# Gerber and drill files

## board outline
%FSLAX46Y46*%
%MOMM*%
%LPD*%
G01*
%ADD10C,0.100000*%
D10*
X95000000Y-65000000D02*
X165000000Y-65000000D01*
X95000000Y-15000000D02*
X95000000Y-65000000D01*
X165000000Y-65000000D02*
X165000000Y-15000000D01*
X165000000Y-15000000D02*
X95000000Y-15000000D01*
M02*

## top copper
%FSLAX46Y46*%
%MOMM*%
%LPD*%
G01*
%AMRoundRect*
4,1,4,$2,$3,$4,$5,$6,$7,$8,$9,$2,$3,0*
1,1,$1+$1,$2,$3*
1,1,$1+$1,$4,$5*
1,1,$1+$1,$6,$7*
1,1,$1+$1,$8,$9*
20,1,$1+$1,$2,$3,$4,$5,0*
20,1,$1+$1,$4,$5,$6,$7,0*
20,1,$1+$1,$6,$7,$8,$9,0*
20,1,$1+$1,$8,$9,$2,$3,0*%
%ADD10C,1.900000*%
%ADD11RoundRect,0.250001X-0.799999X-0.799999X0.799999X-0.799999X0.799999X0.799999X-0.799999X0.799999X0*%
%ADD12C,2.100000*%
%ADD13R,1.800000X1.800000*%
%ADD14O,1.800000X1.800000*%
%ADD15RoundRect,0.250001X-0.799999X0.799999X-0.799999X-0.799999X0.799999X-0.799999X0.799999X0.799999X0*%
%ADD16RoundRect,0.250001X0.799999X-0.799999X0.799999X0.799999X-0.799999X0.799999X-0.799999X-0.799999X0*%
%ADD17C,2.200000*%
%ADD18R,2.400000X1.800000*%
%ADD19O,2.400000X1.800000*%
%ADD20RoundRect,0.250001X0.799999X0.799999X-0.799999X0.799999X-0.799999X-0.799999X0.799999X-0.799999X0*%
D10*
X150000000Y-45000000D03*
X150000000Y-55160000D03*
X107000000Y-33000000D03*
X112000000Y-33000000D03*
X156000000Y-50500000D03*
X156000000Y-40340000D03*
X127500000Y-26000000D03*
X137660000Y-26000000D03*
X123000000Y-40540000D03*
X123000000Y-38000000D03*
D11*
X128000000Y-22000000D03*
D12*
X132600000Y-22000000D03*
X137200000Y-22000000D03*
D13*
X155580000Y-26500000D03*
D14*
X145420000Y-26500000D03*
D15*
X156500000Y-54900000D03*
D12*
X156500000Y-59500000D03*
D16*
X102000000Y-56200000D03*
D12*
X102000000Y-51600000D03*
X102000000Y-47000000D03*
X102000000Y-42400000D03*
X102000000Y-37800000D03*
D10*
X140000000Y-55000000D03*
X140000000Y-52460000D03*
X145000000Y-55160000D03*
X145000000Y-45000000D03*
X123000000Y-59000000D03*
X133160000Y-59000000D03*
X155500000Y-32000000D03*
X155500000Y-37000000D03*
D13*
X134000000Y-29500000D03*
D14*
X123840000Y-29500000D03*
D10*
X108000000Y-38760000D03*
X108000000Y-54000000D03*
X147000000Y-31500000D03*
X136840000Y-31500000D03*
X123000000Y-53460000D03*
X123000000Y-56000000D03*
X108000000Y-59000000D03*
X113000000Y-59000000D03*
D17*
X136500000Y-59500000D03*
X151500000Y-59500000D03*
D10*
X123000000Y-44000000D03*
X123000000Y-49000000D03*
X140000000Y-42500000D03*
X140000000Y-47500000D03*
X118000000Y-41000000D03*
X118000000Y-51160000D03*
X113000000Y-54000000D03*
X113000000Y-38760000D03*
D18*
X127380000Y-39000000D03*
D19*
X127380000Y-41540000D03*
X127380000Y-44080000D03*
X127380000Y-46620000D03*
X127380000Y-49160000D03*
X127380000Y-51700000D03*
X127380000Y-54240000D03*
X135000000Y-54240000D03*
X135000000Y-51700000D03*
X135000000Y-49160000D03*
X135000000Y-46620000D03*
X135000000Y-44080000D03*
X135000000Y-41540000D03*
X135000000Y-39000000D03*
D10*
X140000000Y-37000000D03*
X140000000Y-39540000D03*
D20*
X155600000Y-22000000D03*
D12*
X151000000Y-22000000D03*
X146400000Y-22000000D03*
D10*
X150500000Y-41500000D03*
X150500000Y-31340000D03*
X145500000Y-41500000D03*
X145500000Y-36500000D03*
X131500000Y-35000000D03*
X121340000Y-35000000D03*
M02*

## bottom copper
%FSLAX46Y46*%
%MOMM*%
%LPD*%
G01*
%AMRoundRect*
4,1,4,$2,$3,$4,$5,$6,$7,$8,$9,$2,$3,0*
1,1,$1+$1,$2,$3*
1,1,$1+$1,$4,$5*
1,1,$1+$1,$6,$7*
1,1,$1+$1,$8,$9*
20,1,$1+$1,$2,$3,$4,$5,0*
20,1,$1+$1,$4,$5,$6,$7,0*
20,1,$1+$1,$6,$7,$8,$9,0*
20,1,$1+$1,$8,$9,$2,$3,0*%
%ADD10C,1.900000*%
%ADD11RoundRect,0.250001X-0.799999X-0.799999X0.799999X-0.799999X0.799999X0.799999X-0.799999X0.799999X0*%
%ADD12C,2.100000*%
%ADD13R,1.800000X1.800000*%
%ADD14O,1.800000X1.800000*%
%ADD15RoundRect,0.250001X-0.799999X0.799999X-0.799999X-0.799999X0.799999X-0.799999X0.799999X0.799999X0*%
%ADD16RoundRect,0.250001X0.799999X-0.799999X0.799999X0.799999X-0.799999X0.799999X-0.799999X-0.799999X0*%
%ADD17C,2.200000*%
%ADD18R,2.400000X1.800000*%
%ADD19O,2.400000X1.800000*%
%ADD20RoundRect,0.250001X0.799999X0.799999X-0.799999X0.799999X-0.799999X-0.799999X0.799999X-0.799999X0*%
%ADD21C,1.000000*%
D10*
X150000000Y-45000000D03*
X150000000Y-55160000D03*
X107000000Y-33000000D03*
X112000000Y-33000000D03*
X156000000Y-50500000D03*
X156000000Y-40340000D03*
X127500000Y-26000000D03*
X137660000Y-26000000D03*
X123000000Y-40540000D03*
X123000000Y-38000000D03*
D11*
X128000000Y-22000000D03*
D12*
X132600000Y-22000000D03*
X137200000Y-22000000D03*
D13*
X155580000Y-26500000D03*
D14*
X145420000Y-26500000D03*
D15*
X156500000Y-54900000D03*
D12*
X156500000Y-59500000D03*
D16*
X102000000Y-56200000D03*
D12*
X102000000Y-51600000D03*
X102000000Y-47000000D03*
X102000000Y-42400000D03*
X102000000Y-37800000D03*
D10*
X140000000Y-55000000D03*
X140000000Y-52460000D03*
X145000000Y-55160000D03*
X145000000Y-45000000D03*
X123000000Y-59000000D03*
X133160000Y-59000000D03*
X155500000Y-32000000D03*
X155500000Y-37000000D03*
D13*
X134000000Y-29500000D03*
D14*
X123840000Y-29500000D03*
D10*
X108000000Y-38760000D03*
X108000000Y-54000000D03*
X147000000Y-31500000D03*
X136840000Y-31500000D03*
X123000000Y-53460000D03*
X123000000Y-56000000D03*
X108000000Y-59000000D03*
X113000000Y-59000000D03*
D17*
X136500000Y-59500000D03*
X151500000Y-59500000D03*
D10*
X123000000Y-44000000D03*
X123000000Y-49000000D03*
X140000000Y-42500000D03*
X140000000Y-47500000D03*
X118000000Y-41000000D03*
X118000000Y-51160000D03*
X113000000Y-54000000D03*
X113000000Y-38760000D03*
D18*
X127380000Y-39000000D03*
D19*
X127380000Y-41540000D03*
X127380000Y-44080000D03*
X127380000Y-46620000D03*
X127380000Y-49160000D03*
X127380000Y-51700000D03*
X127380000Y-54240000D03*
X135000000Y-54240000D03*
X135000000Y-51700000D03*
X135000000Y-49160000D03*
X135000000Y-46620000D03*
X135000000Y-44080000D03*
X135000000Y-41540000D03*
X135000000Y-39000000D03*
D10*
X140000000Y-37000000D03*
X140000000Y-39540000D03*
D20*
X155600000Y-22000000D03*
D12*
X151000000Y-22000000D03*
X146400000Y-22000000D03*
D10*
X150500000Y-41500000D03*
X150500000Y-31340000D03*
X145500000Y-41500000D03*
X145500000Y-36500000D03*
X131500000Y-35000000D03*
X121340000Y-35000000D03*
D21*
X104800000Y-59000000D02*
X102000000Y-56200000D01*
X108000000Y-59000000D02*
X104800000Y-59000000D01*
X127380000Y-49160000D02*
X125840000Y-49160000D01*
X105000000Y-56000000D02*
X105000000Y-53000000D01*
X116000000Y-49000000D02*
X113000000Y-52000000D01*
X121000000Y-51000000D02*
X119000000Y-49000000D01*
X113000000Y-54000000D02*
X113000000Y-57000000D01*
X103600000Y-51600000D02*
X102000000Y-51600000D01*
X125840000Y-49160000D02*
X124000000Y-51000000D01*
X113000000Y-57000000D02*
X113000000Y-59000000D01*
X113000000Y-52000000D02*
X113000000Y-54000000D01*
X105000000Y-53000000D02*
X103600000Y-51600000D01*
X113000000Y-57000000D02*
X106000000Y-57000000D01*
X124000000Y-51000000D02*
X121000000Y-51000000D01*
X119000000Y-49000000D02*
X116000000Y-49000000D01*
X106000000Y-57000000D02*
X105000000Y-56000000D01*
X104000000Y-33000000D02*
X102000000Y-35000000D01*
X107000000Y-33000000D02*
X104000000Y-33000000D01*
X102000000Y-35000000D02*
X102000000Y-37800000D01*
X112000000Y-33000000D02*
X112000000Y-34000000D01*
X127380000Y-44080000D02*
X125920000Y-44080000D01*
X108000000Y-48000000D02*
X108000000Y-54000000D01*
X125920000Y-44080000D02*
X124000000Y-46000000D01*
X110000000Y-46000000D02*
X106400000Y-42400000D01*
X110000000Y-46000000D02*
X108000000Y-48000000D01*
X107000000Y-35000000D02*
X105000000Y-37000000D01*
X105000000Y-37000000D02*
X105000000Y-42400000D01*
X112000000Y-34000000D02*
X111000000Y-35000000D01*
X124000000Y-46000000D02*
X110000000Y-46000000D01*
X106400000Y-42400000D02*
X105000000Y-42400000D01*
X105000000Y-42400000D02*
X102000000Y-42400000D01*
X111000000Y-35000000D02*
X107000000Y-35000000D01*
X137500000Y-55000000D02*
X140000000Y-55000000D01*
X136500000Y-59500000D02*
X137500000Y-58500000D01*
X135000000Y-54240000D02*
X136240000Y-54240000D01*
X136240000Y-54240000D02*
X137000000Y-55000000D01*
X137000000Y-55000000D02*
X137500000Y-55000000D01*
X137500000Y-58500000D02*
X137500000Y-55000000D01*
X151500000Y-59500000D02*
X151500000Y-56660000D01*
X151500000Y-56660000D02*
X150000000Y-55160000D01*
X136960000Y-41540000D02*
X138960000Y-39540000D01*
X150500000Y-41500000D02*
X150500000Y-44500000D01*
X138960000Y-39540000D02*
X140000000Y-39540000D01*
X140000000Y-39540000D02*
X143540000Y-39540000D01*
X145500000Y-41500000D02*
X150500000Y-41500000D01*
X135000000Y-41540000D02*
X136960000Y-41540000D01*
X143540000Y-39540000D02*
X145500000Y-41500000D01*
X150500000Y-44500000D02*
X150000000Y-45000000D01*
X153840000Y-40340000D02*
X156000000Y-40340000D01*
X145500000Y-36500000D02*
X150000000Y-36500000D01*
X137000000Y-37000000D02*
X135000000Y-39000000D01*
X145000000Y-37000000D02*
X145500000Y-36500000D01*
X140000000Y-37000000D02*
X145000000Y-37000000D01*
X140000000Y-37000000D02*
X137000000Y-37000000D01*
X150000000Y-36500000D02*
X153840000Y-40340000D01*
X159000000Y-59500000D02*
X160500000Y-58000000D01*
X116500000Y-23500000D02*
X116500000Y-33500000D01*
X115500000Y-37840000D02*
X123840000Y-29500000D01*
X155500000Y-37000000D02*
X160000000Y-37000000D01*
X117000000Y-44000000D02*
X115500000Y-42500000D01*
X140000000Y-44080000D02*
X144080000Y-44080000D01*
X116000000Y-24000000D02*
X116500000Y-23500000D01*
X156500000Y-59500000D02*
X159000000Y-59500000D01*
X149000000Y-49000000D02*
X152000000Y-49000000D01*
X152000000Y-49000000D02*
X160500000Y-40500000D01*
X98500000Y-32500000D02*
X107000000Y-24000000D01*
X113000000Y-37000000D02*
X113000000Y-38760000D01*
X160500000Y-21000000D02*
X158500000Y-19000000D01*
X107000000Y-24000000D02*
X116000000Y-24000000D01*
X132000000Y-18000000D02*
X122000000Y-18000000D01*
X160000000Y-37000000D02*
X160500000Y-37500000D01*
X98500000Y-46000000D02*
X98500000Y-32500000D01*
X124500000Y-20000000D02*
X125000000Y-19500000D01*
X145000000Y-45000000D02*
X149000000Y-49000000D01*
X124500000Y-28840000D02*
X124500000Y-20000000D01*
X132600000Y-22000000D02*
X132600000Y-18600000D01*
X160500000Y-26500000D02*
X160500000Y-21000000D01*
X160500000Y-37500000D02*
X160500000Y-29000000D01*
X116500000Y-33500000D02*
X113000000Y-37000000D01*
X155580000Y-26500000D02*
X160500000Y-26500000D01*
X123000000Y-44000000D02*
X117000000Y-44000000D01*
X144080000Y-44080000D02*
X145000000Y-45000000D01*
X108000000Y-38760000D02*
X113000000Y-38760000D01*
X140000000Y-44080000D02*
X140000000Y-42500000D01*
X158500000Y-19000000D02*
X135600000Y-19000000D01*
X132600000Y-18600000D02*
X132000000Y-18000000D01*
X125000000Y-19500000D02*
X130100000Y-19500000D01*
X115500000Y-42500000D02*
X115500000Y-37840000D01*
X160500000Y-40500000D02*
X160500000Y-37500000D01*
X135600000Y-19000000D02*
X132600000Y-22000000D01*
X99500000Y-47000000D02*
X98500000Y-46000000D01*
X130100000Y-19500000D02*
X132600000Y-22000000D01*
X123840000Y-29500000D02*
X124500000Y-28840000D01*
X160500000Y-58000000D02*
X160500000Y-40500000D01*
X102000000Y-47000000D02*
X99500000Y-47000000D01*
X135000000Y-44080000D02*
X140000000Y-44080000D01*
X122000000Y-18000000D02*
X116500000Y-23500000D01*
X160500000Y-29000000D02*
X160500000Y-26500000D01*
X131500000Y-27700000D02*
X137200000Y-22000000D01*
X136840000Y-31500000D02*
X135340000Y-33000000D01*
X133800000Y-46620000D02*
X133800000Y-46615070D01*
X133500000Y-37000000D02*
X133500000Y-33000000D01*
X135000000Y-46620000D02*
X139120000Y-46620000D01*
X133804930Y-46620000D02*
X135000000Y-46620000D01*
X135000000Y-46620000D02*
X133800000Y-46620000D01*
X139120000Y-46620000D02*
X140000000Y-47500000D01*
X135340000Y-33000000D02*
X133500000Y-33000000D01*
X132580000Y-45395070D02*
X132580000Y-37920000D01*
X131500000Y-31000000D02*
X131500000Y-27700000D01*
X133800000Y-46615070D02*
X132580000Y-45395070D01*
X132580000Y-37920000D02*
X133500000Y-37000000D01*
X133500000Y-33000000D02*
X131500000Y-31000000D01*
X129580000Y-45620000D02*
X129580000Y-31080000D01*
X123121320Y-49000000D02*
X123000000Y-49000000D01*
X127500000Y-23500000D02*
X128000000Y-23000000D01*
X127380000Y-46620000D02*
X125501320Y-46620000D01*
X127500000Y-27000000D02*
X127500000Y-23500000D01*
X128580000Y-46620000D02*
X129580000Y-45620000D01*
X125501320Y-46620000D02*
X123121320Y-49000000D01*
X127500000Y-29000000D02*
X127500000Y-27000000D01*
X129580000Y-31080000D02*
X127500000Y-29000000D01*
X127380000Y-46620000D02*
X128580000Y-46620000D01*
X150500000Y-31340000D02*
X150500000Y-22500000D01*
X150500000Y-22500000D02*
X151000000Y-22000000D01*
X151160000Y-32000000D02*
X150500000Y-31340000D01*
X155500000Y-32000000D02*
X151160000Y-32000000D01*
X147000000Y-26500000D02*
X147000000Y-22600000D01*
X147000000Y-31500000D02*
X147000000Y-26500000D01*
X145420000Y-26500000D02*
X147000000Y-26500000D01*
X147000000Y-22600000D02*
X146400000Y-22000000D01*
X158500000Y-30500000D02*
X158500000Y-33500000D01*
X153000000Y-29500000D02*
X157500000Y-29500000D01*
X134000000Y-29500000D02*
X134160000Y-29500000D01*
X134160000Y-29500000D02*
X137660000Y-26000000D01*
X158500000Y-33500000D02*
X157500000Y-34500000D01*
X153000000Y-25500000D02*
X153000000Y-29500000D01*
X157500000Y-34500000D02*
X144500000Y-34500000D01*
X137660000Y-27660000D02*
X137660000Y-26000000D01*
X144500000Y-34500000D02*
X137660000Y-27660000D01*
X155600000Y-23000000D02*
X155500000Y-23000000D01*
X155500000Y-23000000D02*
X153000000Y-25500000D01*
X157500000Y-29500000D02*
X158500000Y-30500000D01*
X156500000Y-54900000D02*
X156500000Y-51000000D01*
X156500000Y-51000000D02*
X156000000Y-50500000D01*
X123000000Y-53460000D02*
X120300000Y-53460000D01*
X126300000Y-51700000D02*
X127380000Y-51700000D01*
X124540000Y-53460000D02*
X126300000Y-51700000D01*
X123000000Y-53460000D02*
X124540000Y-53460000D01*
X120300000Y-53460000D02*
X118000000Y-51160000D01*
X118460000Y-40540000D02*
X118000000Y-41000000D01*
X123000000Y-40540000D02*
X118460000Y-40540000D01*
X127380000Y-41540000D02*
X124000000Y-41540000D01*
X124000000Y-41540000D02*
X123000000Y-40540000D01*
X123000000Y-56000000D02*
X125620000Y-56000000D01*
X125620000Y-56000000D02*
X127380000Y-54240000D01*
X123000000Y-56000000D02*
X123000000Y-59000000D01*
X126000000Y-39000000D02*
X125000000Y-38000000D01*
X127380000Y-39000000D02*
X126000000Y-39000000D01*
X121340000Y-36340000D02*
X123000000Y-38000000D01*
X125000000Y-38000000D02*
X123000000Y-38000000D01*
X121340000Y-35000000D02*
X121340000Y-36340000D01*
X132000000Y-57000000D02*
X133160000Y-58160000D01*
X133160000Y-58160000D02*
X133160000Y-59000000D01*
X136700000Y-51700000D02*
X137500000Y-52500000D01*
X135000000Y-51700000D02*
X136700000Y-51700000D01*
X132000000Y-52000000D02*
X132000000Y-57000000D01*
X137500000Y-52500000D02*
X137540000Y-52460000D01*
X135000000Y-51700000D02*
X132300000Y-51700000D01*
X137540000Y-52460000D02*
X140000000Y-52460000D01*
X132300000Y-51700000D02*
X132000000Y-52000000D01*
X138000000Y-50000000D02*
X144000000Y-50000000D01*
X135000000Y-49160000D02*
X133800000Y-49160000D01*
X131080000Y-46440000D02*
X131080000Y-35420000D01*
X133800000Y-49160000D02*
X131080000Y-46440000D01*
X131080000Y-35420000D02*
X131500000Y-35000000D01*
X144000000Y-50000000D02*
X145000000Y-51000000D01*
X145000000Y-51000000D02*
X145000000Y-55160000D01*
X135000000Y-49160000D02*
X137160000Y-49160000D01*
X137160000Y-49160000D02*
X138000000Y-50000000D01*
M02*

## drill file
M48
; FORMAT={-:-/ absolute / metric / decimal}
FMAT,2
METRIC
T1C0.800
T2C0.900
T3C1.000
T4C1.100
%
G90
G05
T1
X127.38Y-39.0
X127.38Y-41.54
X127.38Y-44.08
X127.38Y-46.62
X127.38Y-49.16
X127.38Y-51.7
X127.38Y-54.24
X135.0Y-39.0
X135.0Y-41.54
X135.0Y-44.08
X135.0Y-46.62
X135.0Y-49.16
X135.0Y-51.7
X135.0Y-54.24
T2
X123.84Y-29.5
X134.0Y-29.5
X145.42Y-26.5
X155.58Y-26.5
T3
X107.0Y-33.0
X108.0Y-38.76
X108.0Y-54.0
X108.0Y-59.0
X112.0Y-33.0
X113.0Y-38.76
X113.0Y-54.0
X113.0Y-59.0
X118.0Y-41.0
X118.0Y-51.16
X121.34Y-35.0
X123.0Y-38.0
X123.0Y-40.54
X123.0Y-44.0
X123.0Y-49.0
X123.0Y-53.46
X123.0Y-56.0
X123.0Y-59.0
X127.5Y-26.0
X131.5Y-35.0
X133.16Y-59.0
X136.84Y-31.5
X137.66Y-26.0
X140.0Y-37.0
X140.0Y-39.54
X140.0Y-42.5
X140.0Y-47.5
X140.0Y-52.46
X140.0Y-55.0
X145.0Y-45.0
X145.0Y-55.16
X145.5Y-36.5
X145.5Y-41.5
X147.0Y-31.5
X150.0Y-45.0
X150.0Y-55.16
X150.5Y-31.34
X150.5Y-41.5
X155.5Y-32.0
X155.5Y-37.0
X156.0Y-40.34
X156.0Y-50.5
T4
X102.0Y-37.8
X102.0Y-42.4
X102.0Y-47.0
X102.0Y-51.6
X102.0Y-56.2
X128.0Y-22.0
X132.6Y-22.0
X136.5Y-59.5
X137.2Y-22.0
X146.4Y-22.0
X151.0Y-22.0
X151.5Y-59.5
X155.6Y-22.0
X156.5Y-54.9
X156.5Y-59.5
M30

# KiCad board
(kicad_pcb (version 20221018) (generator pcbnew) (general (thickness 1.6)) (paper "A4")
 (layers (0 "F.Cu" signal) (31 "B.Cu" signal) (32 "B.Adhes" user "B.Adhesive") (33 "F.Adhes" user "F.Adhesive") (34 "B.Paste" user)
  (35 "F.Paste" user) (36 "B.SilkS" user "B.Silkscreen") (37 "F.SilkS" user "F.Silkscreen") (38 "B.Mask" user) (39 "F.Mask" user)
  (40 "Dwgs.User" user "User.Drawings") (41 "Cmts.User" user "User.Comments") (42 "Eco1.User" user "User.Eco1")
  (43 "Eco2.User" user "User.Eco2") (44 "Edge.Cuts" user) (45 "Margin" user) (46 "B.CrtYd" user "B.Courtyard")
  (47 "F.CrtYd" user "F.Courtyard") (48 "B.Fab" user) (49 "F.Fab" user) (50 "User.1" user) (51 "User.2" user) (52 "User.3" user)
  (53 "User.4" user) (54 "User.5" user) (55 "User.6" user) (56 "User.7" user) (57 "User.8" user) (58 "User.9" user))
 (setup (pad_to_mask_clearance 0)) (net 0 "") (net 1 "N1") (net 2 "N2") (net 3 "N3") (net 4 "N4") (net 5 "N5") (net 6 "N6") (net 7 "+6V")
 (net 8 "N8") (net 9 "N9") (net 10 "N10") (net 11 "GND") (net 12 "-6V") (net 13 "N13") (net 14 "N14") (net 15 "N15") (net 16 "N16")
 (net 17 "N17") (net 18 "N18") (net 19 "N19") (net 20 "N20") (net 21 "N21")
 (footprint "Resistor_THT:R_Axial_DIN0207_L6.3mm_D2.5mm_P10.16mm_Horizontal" (layer "F.Cu") (at 150 45 -90)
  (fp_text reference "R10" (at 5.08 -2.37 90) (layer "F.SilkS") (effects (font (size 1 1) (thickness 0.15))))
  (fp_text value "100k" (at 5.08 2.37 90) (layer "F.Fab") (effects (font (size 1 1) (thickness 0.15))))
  (pad "1" thru_hole circle (at 0 0 270) (size 1.9 1.9) (drill 1) (layers "*.Cu" "*.Mask") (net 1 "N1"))
  (pad "2" thru_hole circle (at 10.16 0 270) (size 1.9 1.9) (drill 1) (layers "*.Cu" "*.Mask") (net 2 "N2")))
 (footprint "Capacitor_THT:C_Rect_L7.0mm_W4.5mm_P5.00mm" (layer "F.Cu") (at 107 33)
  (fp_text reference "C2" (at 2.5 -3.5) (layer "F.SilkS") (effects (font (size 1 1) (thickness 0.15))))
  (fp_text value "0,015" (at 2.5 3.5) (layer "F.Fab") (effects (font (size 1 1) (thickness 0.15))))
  (pad "1" thru_hole circle (at 0 0) (size 1.9 1.9) (drill 1) (layers "*.Cu" "*.Mask") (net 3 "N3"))
  (pad "2" thru_hole circle (at 5 0) (size 1.9 1.9) (drill 1) (layers "*.Cu" "*.Mask") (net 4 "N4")))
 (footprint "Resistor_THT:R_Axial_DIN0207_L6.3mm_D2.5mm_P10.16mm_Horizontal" (layer "F.Cu") (at 156 50.5 90)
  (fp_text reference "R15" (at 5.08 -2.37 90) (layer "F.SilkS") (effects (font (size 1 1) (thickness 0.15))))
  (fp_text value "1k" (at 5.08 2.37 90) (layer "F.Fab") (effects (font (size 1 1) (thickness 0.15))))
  (pad "1" thru_hole circle (at 0 0 90) (size 1.9 1.9) (drill 1) (layers "*.Cu" "*.Mask") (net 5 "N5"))
  (pad "2" thru_hole circle (at 10.16 0 90) (size 1.9 1.9) (drill 1) (layers "*.Cu" "*.Mask") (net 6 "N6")))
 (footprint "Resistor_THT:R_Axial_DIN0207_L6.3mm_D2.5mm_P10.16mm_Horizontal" (layer "F.Cu") (at 127.5 26)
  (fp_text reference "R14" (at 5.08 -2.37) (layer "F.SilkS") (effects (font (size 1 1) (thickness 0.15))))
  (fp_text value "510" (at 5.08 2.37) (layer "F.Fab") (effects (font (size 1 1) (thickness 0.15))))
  (pad "1" thru_hole circle (at 0 0) (size 1.9 1.9) (drill 1) (layers "*.Cu" "*.Mask") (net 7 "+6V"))
  (pad "2" thru_hole circle (at 10.16 0) (size 1.9 1.9) (drill 1) (layers "*.Cu" "*.Mask") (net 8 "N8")))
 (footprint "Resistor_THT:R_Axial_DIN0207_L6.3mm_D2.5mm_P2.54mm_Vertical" (layer "F.Cu") (at 123 40.54 90)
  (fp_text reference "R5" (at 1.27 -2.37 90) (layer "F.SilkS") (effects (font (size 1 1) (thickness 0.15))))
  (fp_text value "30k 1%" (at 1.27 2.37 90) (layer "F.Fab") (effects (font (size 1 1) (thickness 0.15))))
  (pad "1" thru_hole circle (at 0 0 90) (size 1.9 1.9) (drill 1) (layers "*.Cu" "*.Mask") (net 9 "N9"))
  (pad "2" thru_hole circle (at 2.54 0 90) (size 1.9 1.9) (drill 1) (layers "*.Cu" "*.Mask") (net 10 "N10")))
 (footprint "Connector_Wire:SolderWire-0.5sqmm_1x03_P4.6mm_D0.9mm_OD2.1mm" (layer "F.Cu") (at 128 22)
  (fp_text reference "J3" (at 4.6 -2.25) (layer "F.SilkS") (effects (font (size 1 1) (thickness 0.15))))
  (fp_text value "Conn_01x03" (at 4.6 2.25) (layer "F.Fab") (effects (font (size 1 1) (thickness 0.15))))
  (pad "1" thru_hole roundrect (at 0 0) (size 2.1 2.1) (drill 1.1) (layers "*.Cu" "*.Mask") (roundrect_rratio 0.119048) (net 7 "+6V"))
  (pad "2" thru_hole circle (at 4.6 0) (size 2.1 2.1) (drill 1.1) (layers "*.Cu" "*.Mask") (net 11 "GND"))
  (pad "3" thru_hole circle (at 9.2 0) (size 2.1 2.1) (drill 1.1) (layers "*.Cu" "*.Mask") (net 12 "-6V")))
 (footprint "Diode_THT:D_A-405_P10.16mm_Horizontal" (layer "F.Cu") (at 155.58 26.5 180)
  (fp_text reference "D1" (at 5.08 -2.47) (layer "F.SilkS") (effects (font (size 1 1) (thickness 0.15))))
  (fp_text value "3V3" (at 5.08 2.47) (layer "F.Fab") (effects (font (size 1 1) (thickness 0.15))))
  (pad "1" thru_hole rect (at 0 0 180) (size 1.8 1.8) (drill 0.9) (layers "*.Cu" "*.Mask") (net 11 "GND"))
  (pad "2" thru_hole oval (at 10.16 0 180) (size 1.8 1.8) (drill 0.9) (layers "*.Cu" "*.Mask") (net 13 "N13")))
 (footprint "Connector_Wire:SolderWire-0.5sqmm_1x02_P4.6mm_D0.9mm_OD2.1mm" (layer "F.Cu") (at 156.5 54.9 -90)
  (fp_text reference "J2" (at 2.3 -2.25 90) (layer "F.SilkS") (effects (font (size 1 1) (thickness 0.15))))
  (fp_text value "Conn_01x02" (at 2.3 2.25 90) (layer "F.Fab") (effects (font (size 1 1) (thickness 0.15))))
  (pad "1" thru_hole roundrect (at 0 0 270) (size 2.1 2.1) (drill 1.1) (layers "*.Cu" "*.Mask") (roundrect_rratio 0.119048) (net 5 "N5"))
  (pad "2" thru_hole circle (at 4.6 0 270) (size 2.1 2.1) (drill 1.1) (layers "*.Cu" "*.Mask") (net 11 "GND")))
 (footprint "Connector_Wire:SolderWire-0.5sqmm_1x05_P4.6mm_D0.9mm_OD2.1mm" (layer "F.Cu") (at 102 56.2 90)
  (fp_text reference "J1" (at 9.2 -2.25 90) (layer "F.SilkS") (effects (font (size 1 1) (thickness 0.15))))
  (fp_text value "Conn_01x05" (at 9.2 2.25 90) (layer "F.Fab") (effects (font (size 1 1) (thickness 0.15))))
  (pad "1" thru_hole roundrect (at 0 0 90) (size 2.1 2.1) (drill 1.1) (layers "*.Cu" "*.Mask") (roundrect_rratio 0.119048) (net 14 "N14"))
  (pad "2" thru_hole circle (at 4.6 0 90) (size 2.1 2.1) (drill 1.1) (layers "*.Cu" "*.Mask") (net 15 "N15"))
  (pad "3" thru_hole circle (at 9.2 0 90) (size 2.1 2.1) (drill 1.1) (layers "*.Cu" "*.Mask") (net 11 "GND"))
  (pad "4" thru_hole circle (at 13.8 0 90) (size 2.1 2.1) (drill 1.1) (layers "*.Cu" "*.Mask") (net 4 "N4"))
  (pad "5" thru_hole circle (at 18.4 0 90) (size 2.1 2.1) (drill 1.1) (layers "*.Cu" "*.Mask") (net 3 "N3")))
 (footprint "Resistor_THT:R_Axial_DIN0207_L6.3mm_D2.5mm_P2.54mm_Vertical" (layer "F.Cu") (at 140 55 90)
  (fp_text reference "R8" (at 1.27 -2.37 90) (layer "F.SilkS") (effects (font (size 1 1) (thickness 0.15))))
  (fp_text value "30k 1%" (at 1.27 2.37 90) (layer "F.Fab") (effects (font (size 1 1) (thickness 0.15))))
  (pad "1" thru_hole circle (at 0 0 90) (size 1.9 1.9) (drill 1) (layers "*.Cu" "*.Mask") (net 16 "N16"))
  (pad "2" thru_hole circle (at 2.54 0 90) (size 1.9 1.9) (drill 1) (layers "*.Cu" "*.Mask") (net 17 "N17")))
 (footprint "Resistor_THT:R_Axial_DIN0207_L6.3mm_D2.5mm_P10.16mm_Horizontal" (layer "F.Cu") (at 145 55.16 90)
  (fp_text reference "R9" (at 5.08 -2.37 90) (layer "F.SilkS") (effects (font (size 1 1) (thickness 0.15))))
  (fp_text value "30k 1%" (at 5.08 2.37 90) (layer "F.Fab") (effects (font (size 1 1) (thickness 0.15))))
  (pad "1" thru_hole circle (at 0 0 90) (size 1.9 1.9) (drill 1) (layers "*.Cu" "*.Mask") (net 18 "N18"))
  (pad "2" thru_hole circle (at 10.16 0 90) (size 1.9 1.9) (drill 1) (layers "*.Cu" "*.Mask") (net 11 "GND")))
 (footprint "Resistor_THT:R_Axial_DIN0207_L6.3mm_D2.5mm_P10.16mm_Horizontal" (layer "F.Cu") (at 123 59)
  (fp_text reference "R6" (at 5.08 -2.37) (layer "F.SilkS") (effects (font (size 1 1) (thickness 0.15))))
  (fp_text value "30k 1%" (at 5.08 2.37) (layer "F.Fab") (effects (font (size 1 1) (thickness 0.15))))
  (pad "1" thru_hole circle (at 0 0) (size 1.9 1.9) (drill 1) (layers "*.Cu" "*.Mask") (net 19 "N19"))
  (pad "2" thru_hole circle (at 10.16 0) (size 1.9 1.9) (drill 1) (layers "*.Cu" "*.Mask") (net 17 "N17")))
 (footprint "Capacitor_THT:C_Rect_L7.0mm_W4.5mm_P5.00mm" (layer "F.Cu") (at 155.5 32 -90)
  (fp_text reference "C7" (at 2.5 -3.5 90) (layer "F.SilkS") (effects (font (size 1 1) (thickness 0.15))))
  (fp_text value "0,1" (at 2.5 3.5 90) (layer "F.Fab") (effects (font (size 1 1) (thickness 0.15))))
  (pad "1" thru_hole circle (at 0 0 270) (size 1.9 1.9) (drill 1) (layers "*.Cu" "*.Mask") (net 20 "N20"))
  (pad "2" thru_hole circle (at 5 0 270) (size 1.9 1.9) (drill 1) (layers "*.Cu" "*.Mask") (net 11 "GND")))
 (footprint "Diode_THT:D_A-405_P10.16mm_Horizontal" (layer "F.Cu") (at 134 29.5 180)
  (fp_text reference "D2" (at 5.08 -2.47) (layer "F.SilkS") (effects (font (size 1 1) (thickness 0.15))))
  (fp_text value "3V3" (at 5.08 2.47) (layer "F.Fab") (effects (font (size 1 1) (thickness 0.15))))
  (pad "1" thru_hole rect (at 0 0 180) (size 1.8 1.8) (drill 0.9) (layers "*.Cu" "*.Mask") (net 8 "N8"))
  (pad "2" thru_hole oval (at 10.16 0 180) (size 1.8 1.8) (drill 0.9) (layers "*.Cu" "*.Mask") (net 11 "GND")))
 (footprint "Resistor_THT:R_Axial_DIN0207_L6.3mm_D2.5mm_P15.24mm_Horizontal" (layer "F.Cu") (at 108 38.76 -90)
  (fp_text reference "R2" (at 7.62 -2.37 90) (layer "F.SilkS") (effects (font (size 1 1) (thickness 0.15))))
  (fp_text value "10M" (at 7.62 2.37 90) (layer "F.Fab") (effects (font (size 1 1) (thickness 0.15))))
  (pad "1" thru_hole circle (at 0 0 270) (size 1.9 1.9) (drill 1) (layers "*.Cu" "*.Mask") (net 11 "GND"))
  (pad "2" thru_hole circle (at 15.24 0 270) (size 1.9 1.9) (drill 1) (layers "*.Cu" "*.Mask") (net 4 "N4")))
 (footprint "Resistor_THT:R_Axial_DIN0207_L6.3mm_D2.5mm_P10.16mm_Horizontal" (layer "F.Cu") (at 147 31.5 180)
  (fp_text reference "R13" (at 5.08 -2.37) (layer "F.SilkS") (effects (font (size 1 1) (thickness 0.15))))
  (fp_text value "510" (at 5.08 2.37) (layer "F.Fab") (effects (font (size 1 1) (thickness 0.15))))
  (pad "1" thru_hole circle (at 0 0 180) (size 1.9 1.9) (drill 1) (layers "*.Cu" "*.Mask") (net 13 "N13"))
  (pad "2" thru_hole circle (at 10.16 0 180) (size 1.9 1.9) (drill 1) (layers "*.Cu" "*.Mask") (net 12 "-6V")))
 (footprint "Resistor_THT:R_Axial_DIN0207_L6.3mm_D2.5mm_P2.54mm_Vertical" (layer "F.Cu") (at 123 53.46 -90)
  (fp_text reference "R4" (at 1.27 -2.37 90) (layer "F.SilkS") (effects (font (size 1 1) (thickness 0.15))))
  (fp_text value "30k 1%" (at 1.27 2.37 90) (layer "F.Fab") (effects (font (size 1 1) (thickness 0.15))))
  (pad "1" thru_hole circle (at 0 0 270) (size 1.9 1.9) (drill 1) (layers "*.Cu" "*.Mask") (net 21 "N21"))
  (pad "2" thru_hole circle (at 2.54 0 270) (size 1.9 1.9) (drill 1) (layers "*.Cu" "*.Mask") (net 19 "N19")))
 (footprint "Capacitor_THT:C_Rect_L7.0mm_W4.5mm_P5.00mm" (layer "F.Cu") (at 108 59)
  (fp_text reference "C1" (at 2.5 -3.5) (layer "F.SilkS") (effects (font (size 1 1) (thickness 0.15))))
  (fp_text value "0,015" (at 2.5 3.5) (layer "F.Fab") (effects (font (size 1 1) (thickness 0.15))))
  (pad "1" thru_hole circle (at 0 0) (size 1.9 1.9) (drill 1) (layers "*.Cu" "*.Mask") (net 14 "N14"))
  (pad "2" thru_hole circle (at 5 0) (size 1.9 1.9) (drill 1) (layers "*.Cu" "*.Mask") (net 15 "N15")))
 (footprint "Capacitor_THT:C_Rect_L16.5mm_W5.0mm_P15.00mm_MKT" (layer "F.Cu") (at 136.5 59.5)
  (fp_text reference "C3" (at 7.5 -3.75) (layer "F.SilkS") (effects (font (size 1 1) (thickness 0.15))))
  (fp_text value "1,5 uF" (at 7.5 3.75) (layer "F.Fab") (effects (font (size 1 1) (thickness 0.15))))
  (pad "1" thru_hole circle (at 0 0) (size 2.2 2.2) (drill 1.1) (layers "*.Cu" "*.Mask") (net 16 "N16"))
  (pad "2" thru_hole circle (at 15 0) (size 2.2 2.2) (drill 1.1) (layers "*.Cu" "*.Mask") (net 2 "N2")))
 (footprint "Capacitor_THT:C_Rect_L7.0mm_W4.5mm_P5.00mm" (layer "F.Cu") (at 123 44 -90)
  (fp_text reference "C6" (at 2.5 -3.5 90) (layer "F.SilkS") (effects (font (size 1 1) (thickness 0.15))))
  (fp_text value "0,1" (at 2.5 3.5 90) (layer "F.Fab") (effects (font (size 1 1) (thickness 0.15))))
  (pad "1" thru_hole circle (at 0 0 270) (size 1.9 1.9) (drill 1) (layers "*.Cu" "*.Mask") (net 11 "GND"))
  (pad "2" thru_hole circle (at 5 0 270) (size 1.9 1.9) (drill 1) (layers "*.Cu" "*.Mask") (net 7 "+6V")))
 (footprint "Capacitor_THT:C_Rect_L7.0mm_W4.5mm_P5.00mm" (layer "F.Cu") (at 140 42.5 -90)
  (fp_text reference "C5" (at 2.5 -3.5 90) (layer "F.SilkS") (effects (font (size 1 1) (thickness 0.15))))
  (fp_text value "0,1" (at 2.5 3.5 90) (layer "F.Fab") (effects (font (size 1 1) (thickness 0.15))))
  (pad "1" thru_hole circle (at 0 0 270) (size 1.9 1.9) (drill 1) (layers "*.Cu" "*.Mask") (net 11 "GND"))
  (pad "2" thru_hole circle (at 5 0 270) (size 1.9 1.9) (drill 1) (layers "*.Cu" "*.Mask") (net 12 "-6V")))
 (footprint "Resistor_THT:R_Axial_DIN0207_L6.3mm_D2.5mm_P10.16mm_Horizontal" (layer "F.Cu") (at 118 41 -90)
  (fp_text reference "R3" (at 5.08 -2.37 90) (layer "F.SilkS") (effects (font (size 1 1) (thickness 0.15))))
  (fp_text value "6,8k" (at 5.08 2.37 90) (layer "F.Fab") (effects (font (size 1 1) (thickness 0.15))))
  (pad "1" thru_hole circle (at 0 0 270) (size 1.9 1.9) (drill 1) (layers "*.Cu" "*.Mask") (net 9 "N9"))
  (pad "2" thru_hole circle (at 10.16 0 270) (size 1.9 1.9) (drill 1) (layers "*.Cu" "*.Mask") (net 21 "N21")))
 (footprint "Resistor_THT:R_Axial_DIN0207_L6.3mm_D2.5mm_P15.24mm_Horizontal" (layer "F.Cu") (at 113 54 90)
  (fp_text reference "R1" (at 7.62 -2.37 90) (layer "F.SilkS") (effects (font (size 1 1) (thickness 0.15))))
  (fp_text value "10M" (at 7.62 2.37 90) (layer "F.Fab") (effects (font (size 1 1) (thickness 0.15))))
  (pad "1" thru_hole circle (at 0 0 90) (size 1.9 1.9) (drill 1) (layers "*.Cu" "*.Mask") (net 15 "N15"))
  (pad "2" thru_hole circle (at 15.24 0 90) (size 1.9 1.9) (drill 1) (layers "*.Cu" "*.Mask") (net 11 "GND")))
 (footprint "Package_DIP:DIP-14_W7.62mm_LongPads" (layer "F.Cu") (at 127.38 39)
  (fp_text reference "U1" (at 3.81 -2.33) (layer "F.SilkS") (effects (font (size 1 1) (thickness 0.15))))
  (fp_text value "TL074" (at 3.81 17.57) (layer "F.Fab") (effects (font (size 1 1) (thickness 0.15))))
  (pad "1" thru_hole rect (at 0 0) (size 2.4 1.8) (drill 0.8) (layers "*.Cu" "*.Mask") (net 10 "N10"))
  (pad "2" thru_hole oval (at 0 2.54) (size 2.4 1.8) (drill 0.8) (layers "*.Cu" "*.Mask") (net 9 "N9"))
  (pad "3" thru_hole oval (at 0 5.08) (size 2.4 1.8) (drill 0.8) (layers "*.Cu" "*.Mask") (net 4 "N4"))
  (pad "4" thru_hole oval (at 0 7.62) (size 2.4 1.8) (drill 0.8) (layers "*.Cu" "*.Mask") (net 7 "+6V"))
  (pad "5" thru_hole oval (at 0 10.16) (size 2.4 1.8) (drill 0.8) (layers "*.Cu" "*.Mask") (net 15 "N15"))
  (pad "6" thru_hole oval (at 0 12.7) (size 2.4 1.8) (drill 0.8) (layers "*.Cu" "*.Mask") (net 21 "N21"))
  (pad "7" thru_hole oval (at 0 15.24) (size 2.4 1.8) (drill 0.8) (layers "*.Cu" "*.Mask") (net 19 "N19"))
  (pad "8" thru_hole oval (at 7.62 15.24) (size 2.4 1.8) (drill 0.8) (layers "*.Cu" "*.Mask") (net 16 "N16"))
  (pad "9" thru_hole oval (at 7.62 12.7) (size 2.4 1.8) (drill 0.8) (layers "*.Cu" "*.Mask") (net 17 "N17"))
  (pad "10" thru_hole oval (at 7.62 10.16) (size 2.4 1.8) (drill 0.8) (layers "*.Cu" "*.Mask") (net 18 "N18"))
  (pad "11" thru_hole oval (at 7.62 7.62) (size 2.4 1.8) (drill 0.8) (layers "*.Cu" "*.Mask") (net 12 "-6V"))
  (pad "12" thru_hole oval (at 7.62 5.08) (size 2.4 1.8) (drill 0.8) (layers "*.Cu" "*.Mask") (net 11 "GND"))
  (pad "13" thru_hole oval (at 7.62 2.54) (size 2.4 1.8) (drill 0.8) (layers "*.Cu" "*.Mask") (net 1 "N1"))
  (pad "14" thru_hole oval (at 7.62 0) (size 2.4 1.8) (drill 0.8) (layers "*.Cu" "*.Mask") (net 6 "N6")))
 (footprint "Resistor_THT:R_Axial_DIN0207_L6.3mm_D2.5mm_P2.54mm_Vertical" (layer "F.Cu") (at 140 37 -90)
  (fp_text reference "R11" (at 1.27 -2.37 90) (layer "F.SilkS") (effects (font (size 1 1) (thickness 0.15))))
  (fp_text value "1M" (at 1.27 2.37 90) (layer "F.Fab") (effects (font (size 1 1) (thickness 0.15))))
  (pad "1" thru_hole circle (at 0 0 270) (size 1.9 1.9) (drill 1) (layers "*.Cu" "*.Mask") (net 6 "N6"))
  (pad "2" thru_hole circle (at 2.54 0 270) (size 1.9 1.9) (drill 1) (layers "*.Cu" "*.Mask") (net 1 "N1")))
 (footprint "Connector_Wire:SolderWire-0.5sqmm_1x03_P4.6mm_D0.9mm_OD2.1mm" (layer "F.Cu") (at 155.6 22 180)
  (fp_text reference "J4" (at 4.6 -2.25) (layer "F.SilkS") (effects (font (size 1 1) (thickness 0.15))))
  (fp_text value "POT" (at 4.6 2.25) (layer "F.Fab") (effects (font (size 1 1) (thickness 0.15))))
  (pad "1" thru_hole roundrect (at 0 0 180) (size 2.1 2.1) (drill 1.1) (layers "*.Cu" "*.Mask") (roundrect_rratio 0.119048) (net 8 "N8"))
  (pad "2" thru_hole circle (at 4.6 0 180) (size 2.1 2.1) (drill 1.1) (layers "*.Cu" "*.Mask") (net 20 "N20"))
  (pad "3" thru_hole circle (at 9.2 0 180) (size 2.1 2.1) (drill 1.1) (layers "*.Cu" "*.Mask") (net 13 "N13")))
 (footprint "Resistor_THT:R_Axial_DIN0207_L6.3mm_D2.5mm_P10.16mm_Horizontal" (layer "F.Cu") (at 150.5 41.5 90)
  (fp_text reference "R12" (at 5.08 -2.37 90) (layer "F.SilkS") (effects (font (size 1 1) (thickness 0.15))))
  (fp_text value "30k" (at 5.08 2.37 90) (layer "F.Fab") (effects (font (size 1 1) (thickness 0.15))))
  (pad "1" thru_hole circle (at 0 0 90) (size 1.9 1.9) (drill 1) (layers "*.Cu" "*.Mask") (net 1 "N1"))
  (pad "2" thru_hole circle (at 10.16 0 90) (size 1.9 1.9) (drill 1) (layers "*.Cu" "*.Mask") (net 20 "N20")))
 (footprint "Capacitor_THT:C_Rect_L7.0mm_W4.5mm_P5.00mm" (layer "F.Cu") (at 145.5 41.5 90)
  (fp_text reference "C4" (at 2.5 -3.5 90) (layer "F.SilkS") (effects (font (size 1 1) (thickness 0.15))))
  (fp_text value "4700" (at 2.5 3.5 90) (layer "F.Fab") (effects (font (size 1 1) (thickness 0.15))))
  (pad "1" thru_hole circle (at 0 0 90) (size 1.9 1.9) (drill 1) (layers "*.Cu" "*.Mask") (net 1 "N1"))
  (pad "2" thru_hole circle (at 5 0 90) (size 1.9 1.9) (drill 1) (layers "*.Cu" "*.Mask") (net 6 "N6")))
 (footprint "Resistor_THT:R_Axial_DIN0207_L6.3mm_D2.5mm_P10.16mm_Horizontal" (layer "F.Cu") (at 131.5 35 180)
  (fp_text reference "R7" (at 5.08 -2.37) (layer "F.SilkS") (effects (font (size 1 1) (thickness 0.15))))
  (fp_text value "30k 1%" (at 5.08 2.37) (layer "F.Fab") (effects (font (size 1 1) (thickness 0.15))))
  (pad "1" thru_hole circle (at 0 0 180) (size 1.9 1.9) (drill 1) (layers "*.Cu" "*.Mask") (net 18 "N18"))
  (pad "2" thru_hole circle (at 10.16 0 180) (size 1.9 1.9) (drill 1) (layers "*.Cu" "*.Mask") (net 10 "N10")))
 (gr_line (start 95 65) (end 165 65) (stroke (width 0.1) (type default)) (layer "Edge.Cuts"))
 (gr_line (start 95 15) (end 95 65) (stroke (width 0.1) (type default)) (layer "Edge.Cuts"))
 (gr_line (start 165 65) (end 165 15) (stroke (width 0.1) (type default)) (layer "Edge.Cuts"))
 (gr_line (start 165 15) (end 95 15) (stroke (width 0.1) (type default)) (layer "Edge.Cuts"))
 (segment (start 104.8 59) (end 102 56.2) (width 1) (layer "B.Cu") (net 14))
 (segment (start 108 59) (end 104.8 59) (width 1) (layer "B.Cu") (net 14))
 (segment (start 127.38 49.16) (end 125.84 49.16) (width 1) (layer "B.Cu") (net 15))
 (segment (start 105 56) (end 105 53) (width 1) (layer "B.Cu") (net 15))
 (segment (start 116 49) (end 113 52) (width 1) (layer "B.Cu") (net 15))
 (segment (start 121 51) (end 119 49) (width 1) (layer "B.Cu") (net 15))
 (segment (start 113 54) (end 113 57) (width 1) (layer "B.Cu") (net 15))
 (segment (start 103.6 51.6) (end 102 51.6) (width 1) (layer "B.Cu") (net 15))
 (segment (start 125.84 49.16) (end 124 51) (width 1) (layer "B.Cu") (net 15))
 (segment (start 113 57) (end 113 59) (width 1) (layer "B.Cu") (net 15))
 (segment (start 113 52) (end 113 54) (width 1) (layer "B.Cu") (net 15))
 (segment (start 105 53) (end 103.6 51.6) (width 1) (layer "B.Cu") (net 15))
 (segment (start 113 57) (end 106 57) (width 1) (layer "B.Cu") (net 15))
 (segment (start 124 51) (end 121 51) (width 1) (layer "B.Cu") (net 15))
 (segment (start 119 49) (end 116 49) (width 1) (layer "B.Cu") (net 15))
 (segment (start 106 57) (end 105 56) (width 1) (layer "B.Cu") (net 15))
 (segment (start 104 33) (end 102 35) (width 1) (layer "B.Cu") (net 3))
 (segment (start 107 33) (end 104 33) (width 1) (layer "B.Cu") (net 3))
 (segment (start 102 35) (end 102 37.8) (width 1) (layer "B.Cu") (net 3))
 (segment (start 112 33) (end 112 34) (width 1) (layer "B.Cu") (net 4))
 (segment (start 127.38 44.08) (end 125.92 44.08) (width 1) (layer "B.Cu") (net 4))
 (segment (start 108 48) (end 108 54) (width 1) (layer "B.Cu") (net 4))
 (segment (start 125.92 44.08) (end 124 46) (width 1) (layer "B.Cu") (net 4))
 (segment (start 110 46) (end 106.4 42.4) (width 1) (layer "B.Cu") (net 4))
 (segment (start 110 46) (end 108 48) (width 1) (layer "B.Cu") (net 4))
 (segment (start 107 35) (end 105 37) (width 1) (layer "B.Cu") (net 4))
 (segment (start 105 37) (end 105 42.4) (width 1) (layer "B.Cu") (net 4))
 (segment (start 112 34) (end 111 35) (width 1) (layer "B.Cu") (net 4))
 (segment (start 124 46) (end 110 46) (width 1) (layer "B.Cu") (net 4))
 (segment (start 106.4 42.4) (end 105 42.4) (width 1) (layer "B.Cu") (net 4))
 (segment (start 105 42.4) (end 102 42.4) (width 1) (layer "B.Cu") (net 4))
 (segment (start 111 35) (end 107 35) (width 1) (layer "B.Cu") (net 4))
 (segment (start 137.5 55) (end 140 55) (width 1) (layer "B.Cu") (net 16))
 (segment (start 136.5 59.5) (end 137.5 58.5) (width 1) (layer "B.Cu") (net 16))
 (segment (start 135 54.24) (end 136.24 54.24) (width 1) (layer "B.Cu") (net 16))
 (segment (start 136.24 54.24) (end 137 55) (width 1) (layer "B.Cu") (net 16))
 (segment (start 137 55) (end 137.5 55) (width 1) (layer "B.Cu") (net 16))
 (segment (start 137.5 58.5) (end 137.5 55) (width 1) (layer "B.Cu") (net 16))
 (segment (start 151.5 59.5) (end 151.5 56.66) (width 1) (layer "B.Cu") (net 2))
 (segment (start 151.5 56.66) (end 150 55.16) (width 1) (layer "B.Cu") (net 2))
 (segment (start 136.96 41.54) (end 138.96 39.54) (width 1) (layer "B.Cu") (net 1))
 (segment (start 150.5 41.5) (end 150.5 44.5) (width 1) (layer "B.Cu") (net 1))
 (segment (start 138.96 39.54) (end 140 39.54) (width 1) (layer "B.Cu") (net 1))
 (segment (start 140 39.54) (end 143.54 39.54) (width 1) (layer "B.Cu") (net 1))
 (segment (start 145.5 41.5) (end 150.5 41.5) (width 1) (layer "B.Cu") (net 1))
 (segment (start 135 41.54) (end 136.96 41.54) (width 1) (layer "B.Cu") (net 1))
 (segment (start 143.54 39.54) (end 145.5 41.5) (width 1) (layer "B.Cu") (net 1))
 (segment (start 150.5 44.5) (end 150 45) (width 1) (layer "B.Cu") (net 1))
 (segment (start 153.84 40.34) (end 156 40.34) (width 1) (layer "B.Cu") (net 6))
 (segment (start 145.5 36.5) (end 150 36.5) (width 1) (layer "B.Cu") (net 6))
 (segment (start 137 37) (end 135 39) (width 1) (layer "B.Cu") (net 6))
 (segment (start 145 37) (end 145.5 36.5) (width 1) (layer "B.Cu") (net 6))
 (segment (start 140 37) (end 145 37) (width 1) (layer "B.Cu") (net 6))
 (segment (start 140 37) (end 137 37) (width 1) (layer "B.Cu") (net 6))
 (segment (start 150 36.5) (end 153.84 40.34) (width 1) (layer "B.Cu") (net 6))
 (segment (start 159 59.5) (end 160.5 58) (width 1) (layer "B.Cu") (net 11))
 (segment (start 116.5 23.5) (end 116.5 33.5) (width 1) (layer "B.Cu") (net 11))
 (segment (start 115.5 37.84) (end 123.84 29.5) (width 1) (layer "B.Cu") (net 11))
 (segment (start 155.5 37) (end 160 37) (width 1) (layer "B.Cu") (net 11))
 (segment (start 117 44) (end 115.5 42.5) (width 1) (layer "B.Cu") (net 11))
 (segment (start 140 44.08) (end 144.08 44.08) (width 1) (layer "B.Cu") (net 11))
 (segment (start 116 24) (end 116.5 23.5) (width 1) (layer "B.Cu") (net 11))
 (segment (start 156.5 59.5) (end 159 59.5) (width 1) (layer "B.Cu") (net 11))
 (segment (start 149 49) (end 152 49) (width 1) (layer "B.Cu") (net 11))
 (segment (start 152 49) (end 160.5 40.5) (width 1) (layer "B.Cu") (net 11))
 (segment (start 98.5 32.5) (end 107 24) (width 1) (layer "B.Cu") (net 11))
 (segment (start 113 37) (end 113 38.76) (width 1) (layer "B.Cu") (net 11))
 (segment (start 160.5 21) (end 158.5 19) (width 1) (layer "B.Cu") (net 11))
 (segment (start 107 24) (end 116 24) (width 1) (layer "B.Cu") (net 11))
 (segment (start 132 18) (end 122 18) (width 1) (layer "B.Cu") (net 11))
 (segment (start 160 37) (end 160.5 37.5) (width 1) (layer "B.Cu") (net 11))
 (segment (start 98.5 46) (end 98.5 32.5) (width 1) (layer "B.Cu") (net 11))
 (segment (start 124.5 20) (end 125 19.5) (width 1) (layer "B.Cu") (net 11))
 (segment (start 145 45) (end 149 49) (width 1) (layer "B.Cu") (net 11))
 (segment (start 124.5 28.84) (end 124.5 20) (width 1) (layer "B.Cu") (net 11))
 (segment (start 132.6 22) (end 132.6 18.6) (width 1) (layer "B.Cu") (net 11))
 (segment (start 160.5 26.5) (end 160.5 21) (width 1) (layer "B.Cu") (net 11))
 (segment (start 160.5 37.5) (end 160.5 29) (width 1) (layer "B.Cu") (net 11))
 (segment (start 116.5 33.5) (end 113 37) (width 1) (layer "B.Cu") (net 11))
 (segment (start 155.58 26.5) (end 160.5 26.5) (width 1) (layer "B.Cu") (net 11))
 (segment (start 123 44) (end 117 44) (width 1) (layer "B.Cu") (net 11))
 (segment (start 144.08 44.08) (end 145 45) (width 1) (layer "B.Cu") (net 11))
 (segment (start 108 38.76) (end 113 38.76) (width 1) (layer "B.Cu") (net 11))
 (segment (start 140 44.08) (end 140 42.5) (width 1) (layer "B.Cu") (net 11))
 (segment (start 158.5 19) (end 135.6 19) (width 1) (layer "B.Cu") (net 11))
 (segment (start 132.6 18.6) (end 132 18) (width 1) (layer "B.Cu") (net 11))
 (segment (start 125 19.5) (end 130.1 19.5) (width 1) (layer "B.Cu") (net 11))
 (segment (start 115.5 42.5) (end 115.5 37.84) (width 1) (layer "B.Cu") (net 11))
 (segment (start 160.5 40.5) (end 160.5 37.5) (width 1) (layer "B.Cu") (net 11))
 (segment (start 135.6 19) (end 132.6 22) (width 1) (layer "B.Cu") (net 11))
 (segment (start 99.5 47) (end 98.5 46) (width 1) (layer "B.Cu") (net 11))
 (segment (start 130.1 19.5) (end 132.6 22) (width 1) (layer "B.Cu") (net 11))
 (segment (start 123.84 29.5) (end 124.5 28.84) (width 1) (layer "B.Cu") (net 11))
 (segment (start 160.5 58) (end 160.5 40.5) (width 1) (layer "B.Cu") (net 11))
 (segment (start 102 47) (end 99.5 47) (width 1) (layer "B.Cu") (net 11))
 (segment (start 135 44.08) (end 140 44.08) (width 1) (layer "B.Cu") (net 11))
 (segment (start 122 18) (end 116.5 23.5) (width 1) (layer "B.Cu") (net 11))
 (segment (start 160.5 29) (end 160.5 26.5) (width 1) (layer "B.Cu") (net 11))
 (segment (start 131.5 27.7) (end 137.2 22) (width 1) (layer "B.Cu") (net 12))
 (segment (start 136.84 31.5) (end 135.34 33) (width 1) (layer "B.Cu") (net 12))
 (segment (start 133.8 46.62) (end 133.8 46.61507) (width 1) (layer "B.Cu") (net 12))
 (segment (start 133.5 37) (end 133.5 33) (width 1) (layer "B.Cu") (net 12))
 (segment (start 135 46.62) (end 139.12 46.62) (width 1) (layer "B.Cu") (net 12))
 (segment (start 133.80493 46.62) (end 135 46.62) (width 1) (layer "B.Cu") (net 12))
 (segment (start 135 46.62) (end 133.8 46.62) (width 1) (layer "B.Cu") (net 12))
 (segment (start 139.12 46.62) (end 140 47.5) (width 1) (layer "B.Cu") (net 12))
 (segment (start 135.34 33) (end 133.5 33) (width 1) (layer "B.Cu") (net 12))
 (segment (start 132.58 45.39507) (end 132.58 37.92) (width 1) (layer "B.Cu") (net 12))
 (segment (start 131.5 31) (end 131.5 27.7) (width 1) (layer "B.Cu") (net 12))
 (segment (start 133.8 46.61507) (end 132.58 45.39507) (width 1) (layer "B.Cu") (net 12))
 (segment (start 132.58 37.92) (end 133.5 37) (width 1) (layer "B.Cu") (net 12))
 (segment (start 133.5 33) (end 131.5 31) (width 1) (layer "B.Cu") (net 12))
 (segment (start 129.58 45.62) (end 129.58 31.08) (width 1) (layer "B.Cu") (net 7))
 (segment (start 123.12132 49) (end 123 49) (width 1) (layer "B.Cu") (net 7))
 (segment (start 127.5 23.5) (end 128 23) (width 1) (layer "B.Cu") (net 7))
 (segment (start 127.38 46.62) (end 125.50132 46.62) (width 1) (layer "B.Cu") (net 7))
 (segment (start 127.5 27) (end 127.5 23.5) (width 1) (layer "B.Cu") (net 7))
 (segment (start 128.58 46.62) (end 129.58 45.62) (width 1) (layer "B.Cu") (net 7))
 (segment (start 125.50132 46.62) (end 123.12132 49) (width 1) (layer "B.Cu") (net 7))
 (segment (start 127.5 29) (end 127.5 27) (width 1) (layer "B.Cu") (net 7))
 (segment (start 129.58 31.08) (end 127.5 29) (width 1) (layer "B.Cu") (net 7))
 (segment (start 127.38 46.62) (end 128.58 46.62) (width 1) (layer "B.Cu") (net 7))
 (segment (start 150.5 31.34) (end 150.5 22.5) (width 1) (layer "B.Cu") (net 20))
 (segment (start 150.5 22.5) (end 151 22) (width 1) (layer "B.Cu") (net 20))
 (segment (start 151.16 32) (end 150.5 31.34) (width 1) (layer "B.Cu") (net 20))
 (segment (start 155.5 32) (end 151.16 32) (width 1) (layer "B.Cu") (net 20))
 (segment (start 147 26.5) (end 147 22.6) (width 1) (layer "B.Cu") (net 13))
 (segment (start 147 31.5) (end 147 26.5) (width 1) (layer "B.Cu") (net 13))
 (segment (start 145.42 26.5) (end 147 26.5) (width 1) (layer "B.Cu") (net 13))
 (segment (start 147 22.6) (end 146.4 22) (width 1) (layer "B.Cu") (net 13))
 (segment (start 158.5 30.5) (end 158.5 33.5) (width 1) (layer "B.Cu") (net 8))
 (segment (start 153 29.5) (end 157.5 29.5) (width 1) (layer "B.Cu") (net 8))
 (segment (start 134 29.5) (end 134.16 29.5) (width 1) (layer "B.Cu") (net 8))
 (segment (start 134.16 29.5) (end 137.66 26) (width 1) (layer "B.Cu") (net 8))
 (segment (start 158.5 33.5) (end 157.5 34.5) (width 1) (layer "B.Cu") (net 8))
 (segment (start 153 25.5) (end 153 29.5) (width 1) (layer "B.Cu") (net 8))
 (segment (start 157.5 34.5) (end 144.5 34.5) (width 1) (layer "B.Cu") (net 8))
 (segment (start 137.66 27.66) (end 137.66 26) (width 1) (layer "B.Cu") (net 8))
 (segment (start 144.5 34.5) (end 137.66 27.66) (width 1) (layer "B.Cu") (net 8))
 (segment (start 155.6 23) (end 155.5 23) (width 1) (layer "B.Cu") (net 8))
 (segment (start 155.5 23) (end 153 25.5) (width 1) (layer "B.Cu") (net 8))
 (segment (start 157.5 29.5) (end 158.5 30.5) (width 1) (layer "B.Cu") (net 8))
 (segment (start 156.5 54.9) (end 156.5 51) (width 1) (layer "B.Cu") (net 5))
 (segment (start 156.5 51) (end 156 50.5) (width 1) (layer "B.Cu") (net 5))
 (segment (start 123 53.46) (end 120.3 53.46) (width 1) (layer "B.Cu") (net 21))
 (segment (start 126.3 51.7) (end 127.38 51.7) (width 1) (layer "B.Cu") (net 21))
 (segment (start 124.54 53.46) (end 126.3 51.7) (width 1) (layer "B.Cu") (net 21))
 (segment (start 123 53.46) (end 124.54 53.46) (width 1) (layer "B.Cu") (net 21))
 (segment (start 120.3 53.46) (end 118 51.16) (width 1) (layer "B.Cu") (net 21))
 (segment (start 118.46 40.54) (end 118 41) (width 1) (layer "B.Cu") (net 9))
 (segment (start 123 40.54) (end 118.46 40.54) (width 1) (layer "B.Cu") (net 9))
 (segment (start 127.38 41.54) (end 124 41.54) (width 1) (layer "B.Cu") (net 9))
 (segment (start 124 41.54) (end 123 40.54) (width 1) (layer "B.Cu") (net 9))
 (segment (start 123 56) (end 125.62 56) (width 1) (layer "B.Cu") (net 19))
 (segment (start 125.62 56) (end 127.38 54.24) (width 1) (layer "B.Cu") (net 19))
 (segment (start 123 56) (end 123 59) (width 1) (layer "B.Cu") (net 19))
 (segment (start 126 39) (end 125 38) (width 1) (layer "B.Cu") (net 10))
 (segment (start 127.38 39) (end 126 39) (width 1) (layer "B.Cu") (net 10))
 (segment (start 121.34 36.34) (end 123 38) (width 1) (layer "B.Cu") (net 10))
 (segment (start 125 38) (end 123 38) (width 1) (layer "B.Cu") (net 10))
 (segment (start 121.34 35) (end 121.34 36.34) (width 1) (layer "B.Cu") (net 10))
 (segment (start 132 57) (end 133.16 58.16) (width 1) (layer "B.Cu") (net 17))
 (segment (start 133.16 58.16) (end 133.16 59) (width 1) (layer "B.Cu") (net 17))
 (segment (start 136.7 51.7) (end 137.5 52.5) (width 1) (layer "B.Cu") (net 17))
 (segment (start 135 51.7) (end 136.7 51.7) (width 1) (layer "B.Cu") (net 17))
 (segment (start 132 52) (end 132 57) (width 1) (layer "B.Cu") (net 17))
 (segment (start 137.5 52.5) (end 137.54 52.46) (width 1) (layer "B.Cu") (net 17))
 (segment (start 135 51.7) (end 132.3 51.7) (width 1) (layer "B.Cu") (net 17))
 (segment (start 137.54 52.46) (end 140 52.46) (width 1) (layer "B.Cu") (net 17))
 (segment (start 132.3 51.7) (end 132 52) (width 1) (layer "B.Cu") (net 17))
 (segment (start 138 50) (end 144 50) (width 1) (layer "B.Cu") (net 18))
 (segment (start 135 49.16) (end 133.8 49.16) (width 1) (layer "B.Cu") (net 18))
 (segment (start 131.08 46.44) (end 131.08 35.42) (width 1) (layer "B.Cu") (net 18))
 (segment (start 133.8 49.16) (end 131.08 46.44) (width 1) (layer "B.Cu") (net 18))
 (segment (start 131.08 35.42) (end 131.5 35) (width 1) (layer "B.Cu") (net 18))
 (segment (start 144 50) (end 145 51) (width 1) (layer "B.Cu") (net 18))
 (segment (start 145 51) (end 145 55.16) (width 1) (layer "B.Cu") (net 18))
 (segment (start 135 49.16) (end 137.16 49.16) (width 1) (layer "B.Cu") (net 18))
 (segment (start 137.16 49.16) (end 138 50) (width 1) (layer "B.Cu") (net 18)))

